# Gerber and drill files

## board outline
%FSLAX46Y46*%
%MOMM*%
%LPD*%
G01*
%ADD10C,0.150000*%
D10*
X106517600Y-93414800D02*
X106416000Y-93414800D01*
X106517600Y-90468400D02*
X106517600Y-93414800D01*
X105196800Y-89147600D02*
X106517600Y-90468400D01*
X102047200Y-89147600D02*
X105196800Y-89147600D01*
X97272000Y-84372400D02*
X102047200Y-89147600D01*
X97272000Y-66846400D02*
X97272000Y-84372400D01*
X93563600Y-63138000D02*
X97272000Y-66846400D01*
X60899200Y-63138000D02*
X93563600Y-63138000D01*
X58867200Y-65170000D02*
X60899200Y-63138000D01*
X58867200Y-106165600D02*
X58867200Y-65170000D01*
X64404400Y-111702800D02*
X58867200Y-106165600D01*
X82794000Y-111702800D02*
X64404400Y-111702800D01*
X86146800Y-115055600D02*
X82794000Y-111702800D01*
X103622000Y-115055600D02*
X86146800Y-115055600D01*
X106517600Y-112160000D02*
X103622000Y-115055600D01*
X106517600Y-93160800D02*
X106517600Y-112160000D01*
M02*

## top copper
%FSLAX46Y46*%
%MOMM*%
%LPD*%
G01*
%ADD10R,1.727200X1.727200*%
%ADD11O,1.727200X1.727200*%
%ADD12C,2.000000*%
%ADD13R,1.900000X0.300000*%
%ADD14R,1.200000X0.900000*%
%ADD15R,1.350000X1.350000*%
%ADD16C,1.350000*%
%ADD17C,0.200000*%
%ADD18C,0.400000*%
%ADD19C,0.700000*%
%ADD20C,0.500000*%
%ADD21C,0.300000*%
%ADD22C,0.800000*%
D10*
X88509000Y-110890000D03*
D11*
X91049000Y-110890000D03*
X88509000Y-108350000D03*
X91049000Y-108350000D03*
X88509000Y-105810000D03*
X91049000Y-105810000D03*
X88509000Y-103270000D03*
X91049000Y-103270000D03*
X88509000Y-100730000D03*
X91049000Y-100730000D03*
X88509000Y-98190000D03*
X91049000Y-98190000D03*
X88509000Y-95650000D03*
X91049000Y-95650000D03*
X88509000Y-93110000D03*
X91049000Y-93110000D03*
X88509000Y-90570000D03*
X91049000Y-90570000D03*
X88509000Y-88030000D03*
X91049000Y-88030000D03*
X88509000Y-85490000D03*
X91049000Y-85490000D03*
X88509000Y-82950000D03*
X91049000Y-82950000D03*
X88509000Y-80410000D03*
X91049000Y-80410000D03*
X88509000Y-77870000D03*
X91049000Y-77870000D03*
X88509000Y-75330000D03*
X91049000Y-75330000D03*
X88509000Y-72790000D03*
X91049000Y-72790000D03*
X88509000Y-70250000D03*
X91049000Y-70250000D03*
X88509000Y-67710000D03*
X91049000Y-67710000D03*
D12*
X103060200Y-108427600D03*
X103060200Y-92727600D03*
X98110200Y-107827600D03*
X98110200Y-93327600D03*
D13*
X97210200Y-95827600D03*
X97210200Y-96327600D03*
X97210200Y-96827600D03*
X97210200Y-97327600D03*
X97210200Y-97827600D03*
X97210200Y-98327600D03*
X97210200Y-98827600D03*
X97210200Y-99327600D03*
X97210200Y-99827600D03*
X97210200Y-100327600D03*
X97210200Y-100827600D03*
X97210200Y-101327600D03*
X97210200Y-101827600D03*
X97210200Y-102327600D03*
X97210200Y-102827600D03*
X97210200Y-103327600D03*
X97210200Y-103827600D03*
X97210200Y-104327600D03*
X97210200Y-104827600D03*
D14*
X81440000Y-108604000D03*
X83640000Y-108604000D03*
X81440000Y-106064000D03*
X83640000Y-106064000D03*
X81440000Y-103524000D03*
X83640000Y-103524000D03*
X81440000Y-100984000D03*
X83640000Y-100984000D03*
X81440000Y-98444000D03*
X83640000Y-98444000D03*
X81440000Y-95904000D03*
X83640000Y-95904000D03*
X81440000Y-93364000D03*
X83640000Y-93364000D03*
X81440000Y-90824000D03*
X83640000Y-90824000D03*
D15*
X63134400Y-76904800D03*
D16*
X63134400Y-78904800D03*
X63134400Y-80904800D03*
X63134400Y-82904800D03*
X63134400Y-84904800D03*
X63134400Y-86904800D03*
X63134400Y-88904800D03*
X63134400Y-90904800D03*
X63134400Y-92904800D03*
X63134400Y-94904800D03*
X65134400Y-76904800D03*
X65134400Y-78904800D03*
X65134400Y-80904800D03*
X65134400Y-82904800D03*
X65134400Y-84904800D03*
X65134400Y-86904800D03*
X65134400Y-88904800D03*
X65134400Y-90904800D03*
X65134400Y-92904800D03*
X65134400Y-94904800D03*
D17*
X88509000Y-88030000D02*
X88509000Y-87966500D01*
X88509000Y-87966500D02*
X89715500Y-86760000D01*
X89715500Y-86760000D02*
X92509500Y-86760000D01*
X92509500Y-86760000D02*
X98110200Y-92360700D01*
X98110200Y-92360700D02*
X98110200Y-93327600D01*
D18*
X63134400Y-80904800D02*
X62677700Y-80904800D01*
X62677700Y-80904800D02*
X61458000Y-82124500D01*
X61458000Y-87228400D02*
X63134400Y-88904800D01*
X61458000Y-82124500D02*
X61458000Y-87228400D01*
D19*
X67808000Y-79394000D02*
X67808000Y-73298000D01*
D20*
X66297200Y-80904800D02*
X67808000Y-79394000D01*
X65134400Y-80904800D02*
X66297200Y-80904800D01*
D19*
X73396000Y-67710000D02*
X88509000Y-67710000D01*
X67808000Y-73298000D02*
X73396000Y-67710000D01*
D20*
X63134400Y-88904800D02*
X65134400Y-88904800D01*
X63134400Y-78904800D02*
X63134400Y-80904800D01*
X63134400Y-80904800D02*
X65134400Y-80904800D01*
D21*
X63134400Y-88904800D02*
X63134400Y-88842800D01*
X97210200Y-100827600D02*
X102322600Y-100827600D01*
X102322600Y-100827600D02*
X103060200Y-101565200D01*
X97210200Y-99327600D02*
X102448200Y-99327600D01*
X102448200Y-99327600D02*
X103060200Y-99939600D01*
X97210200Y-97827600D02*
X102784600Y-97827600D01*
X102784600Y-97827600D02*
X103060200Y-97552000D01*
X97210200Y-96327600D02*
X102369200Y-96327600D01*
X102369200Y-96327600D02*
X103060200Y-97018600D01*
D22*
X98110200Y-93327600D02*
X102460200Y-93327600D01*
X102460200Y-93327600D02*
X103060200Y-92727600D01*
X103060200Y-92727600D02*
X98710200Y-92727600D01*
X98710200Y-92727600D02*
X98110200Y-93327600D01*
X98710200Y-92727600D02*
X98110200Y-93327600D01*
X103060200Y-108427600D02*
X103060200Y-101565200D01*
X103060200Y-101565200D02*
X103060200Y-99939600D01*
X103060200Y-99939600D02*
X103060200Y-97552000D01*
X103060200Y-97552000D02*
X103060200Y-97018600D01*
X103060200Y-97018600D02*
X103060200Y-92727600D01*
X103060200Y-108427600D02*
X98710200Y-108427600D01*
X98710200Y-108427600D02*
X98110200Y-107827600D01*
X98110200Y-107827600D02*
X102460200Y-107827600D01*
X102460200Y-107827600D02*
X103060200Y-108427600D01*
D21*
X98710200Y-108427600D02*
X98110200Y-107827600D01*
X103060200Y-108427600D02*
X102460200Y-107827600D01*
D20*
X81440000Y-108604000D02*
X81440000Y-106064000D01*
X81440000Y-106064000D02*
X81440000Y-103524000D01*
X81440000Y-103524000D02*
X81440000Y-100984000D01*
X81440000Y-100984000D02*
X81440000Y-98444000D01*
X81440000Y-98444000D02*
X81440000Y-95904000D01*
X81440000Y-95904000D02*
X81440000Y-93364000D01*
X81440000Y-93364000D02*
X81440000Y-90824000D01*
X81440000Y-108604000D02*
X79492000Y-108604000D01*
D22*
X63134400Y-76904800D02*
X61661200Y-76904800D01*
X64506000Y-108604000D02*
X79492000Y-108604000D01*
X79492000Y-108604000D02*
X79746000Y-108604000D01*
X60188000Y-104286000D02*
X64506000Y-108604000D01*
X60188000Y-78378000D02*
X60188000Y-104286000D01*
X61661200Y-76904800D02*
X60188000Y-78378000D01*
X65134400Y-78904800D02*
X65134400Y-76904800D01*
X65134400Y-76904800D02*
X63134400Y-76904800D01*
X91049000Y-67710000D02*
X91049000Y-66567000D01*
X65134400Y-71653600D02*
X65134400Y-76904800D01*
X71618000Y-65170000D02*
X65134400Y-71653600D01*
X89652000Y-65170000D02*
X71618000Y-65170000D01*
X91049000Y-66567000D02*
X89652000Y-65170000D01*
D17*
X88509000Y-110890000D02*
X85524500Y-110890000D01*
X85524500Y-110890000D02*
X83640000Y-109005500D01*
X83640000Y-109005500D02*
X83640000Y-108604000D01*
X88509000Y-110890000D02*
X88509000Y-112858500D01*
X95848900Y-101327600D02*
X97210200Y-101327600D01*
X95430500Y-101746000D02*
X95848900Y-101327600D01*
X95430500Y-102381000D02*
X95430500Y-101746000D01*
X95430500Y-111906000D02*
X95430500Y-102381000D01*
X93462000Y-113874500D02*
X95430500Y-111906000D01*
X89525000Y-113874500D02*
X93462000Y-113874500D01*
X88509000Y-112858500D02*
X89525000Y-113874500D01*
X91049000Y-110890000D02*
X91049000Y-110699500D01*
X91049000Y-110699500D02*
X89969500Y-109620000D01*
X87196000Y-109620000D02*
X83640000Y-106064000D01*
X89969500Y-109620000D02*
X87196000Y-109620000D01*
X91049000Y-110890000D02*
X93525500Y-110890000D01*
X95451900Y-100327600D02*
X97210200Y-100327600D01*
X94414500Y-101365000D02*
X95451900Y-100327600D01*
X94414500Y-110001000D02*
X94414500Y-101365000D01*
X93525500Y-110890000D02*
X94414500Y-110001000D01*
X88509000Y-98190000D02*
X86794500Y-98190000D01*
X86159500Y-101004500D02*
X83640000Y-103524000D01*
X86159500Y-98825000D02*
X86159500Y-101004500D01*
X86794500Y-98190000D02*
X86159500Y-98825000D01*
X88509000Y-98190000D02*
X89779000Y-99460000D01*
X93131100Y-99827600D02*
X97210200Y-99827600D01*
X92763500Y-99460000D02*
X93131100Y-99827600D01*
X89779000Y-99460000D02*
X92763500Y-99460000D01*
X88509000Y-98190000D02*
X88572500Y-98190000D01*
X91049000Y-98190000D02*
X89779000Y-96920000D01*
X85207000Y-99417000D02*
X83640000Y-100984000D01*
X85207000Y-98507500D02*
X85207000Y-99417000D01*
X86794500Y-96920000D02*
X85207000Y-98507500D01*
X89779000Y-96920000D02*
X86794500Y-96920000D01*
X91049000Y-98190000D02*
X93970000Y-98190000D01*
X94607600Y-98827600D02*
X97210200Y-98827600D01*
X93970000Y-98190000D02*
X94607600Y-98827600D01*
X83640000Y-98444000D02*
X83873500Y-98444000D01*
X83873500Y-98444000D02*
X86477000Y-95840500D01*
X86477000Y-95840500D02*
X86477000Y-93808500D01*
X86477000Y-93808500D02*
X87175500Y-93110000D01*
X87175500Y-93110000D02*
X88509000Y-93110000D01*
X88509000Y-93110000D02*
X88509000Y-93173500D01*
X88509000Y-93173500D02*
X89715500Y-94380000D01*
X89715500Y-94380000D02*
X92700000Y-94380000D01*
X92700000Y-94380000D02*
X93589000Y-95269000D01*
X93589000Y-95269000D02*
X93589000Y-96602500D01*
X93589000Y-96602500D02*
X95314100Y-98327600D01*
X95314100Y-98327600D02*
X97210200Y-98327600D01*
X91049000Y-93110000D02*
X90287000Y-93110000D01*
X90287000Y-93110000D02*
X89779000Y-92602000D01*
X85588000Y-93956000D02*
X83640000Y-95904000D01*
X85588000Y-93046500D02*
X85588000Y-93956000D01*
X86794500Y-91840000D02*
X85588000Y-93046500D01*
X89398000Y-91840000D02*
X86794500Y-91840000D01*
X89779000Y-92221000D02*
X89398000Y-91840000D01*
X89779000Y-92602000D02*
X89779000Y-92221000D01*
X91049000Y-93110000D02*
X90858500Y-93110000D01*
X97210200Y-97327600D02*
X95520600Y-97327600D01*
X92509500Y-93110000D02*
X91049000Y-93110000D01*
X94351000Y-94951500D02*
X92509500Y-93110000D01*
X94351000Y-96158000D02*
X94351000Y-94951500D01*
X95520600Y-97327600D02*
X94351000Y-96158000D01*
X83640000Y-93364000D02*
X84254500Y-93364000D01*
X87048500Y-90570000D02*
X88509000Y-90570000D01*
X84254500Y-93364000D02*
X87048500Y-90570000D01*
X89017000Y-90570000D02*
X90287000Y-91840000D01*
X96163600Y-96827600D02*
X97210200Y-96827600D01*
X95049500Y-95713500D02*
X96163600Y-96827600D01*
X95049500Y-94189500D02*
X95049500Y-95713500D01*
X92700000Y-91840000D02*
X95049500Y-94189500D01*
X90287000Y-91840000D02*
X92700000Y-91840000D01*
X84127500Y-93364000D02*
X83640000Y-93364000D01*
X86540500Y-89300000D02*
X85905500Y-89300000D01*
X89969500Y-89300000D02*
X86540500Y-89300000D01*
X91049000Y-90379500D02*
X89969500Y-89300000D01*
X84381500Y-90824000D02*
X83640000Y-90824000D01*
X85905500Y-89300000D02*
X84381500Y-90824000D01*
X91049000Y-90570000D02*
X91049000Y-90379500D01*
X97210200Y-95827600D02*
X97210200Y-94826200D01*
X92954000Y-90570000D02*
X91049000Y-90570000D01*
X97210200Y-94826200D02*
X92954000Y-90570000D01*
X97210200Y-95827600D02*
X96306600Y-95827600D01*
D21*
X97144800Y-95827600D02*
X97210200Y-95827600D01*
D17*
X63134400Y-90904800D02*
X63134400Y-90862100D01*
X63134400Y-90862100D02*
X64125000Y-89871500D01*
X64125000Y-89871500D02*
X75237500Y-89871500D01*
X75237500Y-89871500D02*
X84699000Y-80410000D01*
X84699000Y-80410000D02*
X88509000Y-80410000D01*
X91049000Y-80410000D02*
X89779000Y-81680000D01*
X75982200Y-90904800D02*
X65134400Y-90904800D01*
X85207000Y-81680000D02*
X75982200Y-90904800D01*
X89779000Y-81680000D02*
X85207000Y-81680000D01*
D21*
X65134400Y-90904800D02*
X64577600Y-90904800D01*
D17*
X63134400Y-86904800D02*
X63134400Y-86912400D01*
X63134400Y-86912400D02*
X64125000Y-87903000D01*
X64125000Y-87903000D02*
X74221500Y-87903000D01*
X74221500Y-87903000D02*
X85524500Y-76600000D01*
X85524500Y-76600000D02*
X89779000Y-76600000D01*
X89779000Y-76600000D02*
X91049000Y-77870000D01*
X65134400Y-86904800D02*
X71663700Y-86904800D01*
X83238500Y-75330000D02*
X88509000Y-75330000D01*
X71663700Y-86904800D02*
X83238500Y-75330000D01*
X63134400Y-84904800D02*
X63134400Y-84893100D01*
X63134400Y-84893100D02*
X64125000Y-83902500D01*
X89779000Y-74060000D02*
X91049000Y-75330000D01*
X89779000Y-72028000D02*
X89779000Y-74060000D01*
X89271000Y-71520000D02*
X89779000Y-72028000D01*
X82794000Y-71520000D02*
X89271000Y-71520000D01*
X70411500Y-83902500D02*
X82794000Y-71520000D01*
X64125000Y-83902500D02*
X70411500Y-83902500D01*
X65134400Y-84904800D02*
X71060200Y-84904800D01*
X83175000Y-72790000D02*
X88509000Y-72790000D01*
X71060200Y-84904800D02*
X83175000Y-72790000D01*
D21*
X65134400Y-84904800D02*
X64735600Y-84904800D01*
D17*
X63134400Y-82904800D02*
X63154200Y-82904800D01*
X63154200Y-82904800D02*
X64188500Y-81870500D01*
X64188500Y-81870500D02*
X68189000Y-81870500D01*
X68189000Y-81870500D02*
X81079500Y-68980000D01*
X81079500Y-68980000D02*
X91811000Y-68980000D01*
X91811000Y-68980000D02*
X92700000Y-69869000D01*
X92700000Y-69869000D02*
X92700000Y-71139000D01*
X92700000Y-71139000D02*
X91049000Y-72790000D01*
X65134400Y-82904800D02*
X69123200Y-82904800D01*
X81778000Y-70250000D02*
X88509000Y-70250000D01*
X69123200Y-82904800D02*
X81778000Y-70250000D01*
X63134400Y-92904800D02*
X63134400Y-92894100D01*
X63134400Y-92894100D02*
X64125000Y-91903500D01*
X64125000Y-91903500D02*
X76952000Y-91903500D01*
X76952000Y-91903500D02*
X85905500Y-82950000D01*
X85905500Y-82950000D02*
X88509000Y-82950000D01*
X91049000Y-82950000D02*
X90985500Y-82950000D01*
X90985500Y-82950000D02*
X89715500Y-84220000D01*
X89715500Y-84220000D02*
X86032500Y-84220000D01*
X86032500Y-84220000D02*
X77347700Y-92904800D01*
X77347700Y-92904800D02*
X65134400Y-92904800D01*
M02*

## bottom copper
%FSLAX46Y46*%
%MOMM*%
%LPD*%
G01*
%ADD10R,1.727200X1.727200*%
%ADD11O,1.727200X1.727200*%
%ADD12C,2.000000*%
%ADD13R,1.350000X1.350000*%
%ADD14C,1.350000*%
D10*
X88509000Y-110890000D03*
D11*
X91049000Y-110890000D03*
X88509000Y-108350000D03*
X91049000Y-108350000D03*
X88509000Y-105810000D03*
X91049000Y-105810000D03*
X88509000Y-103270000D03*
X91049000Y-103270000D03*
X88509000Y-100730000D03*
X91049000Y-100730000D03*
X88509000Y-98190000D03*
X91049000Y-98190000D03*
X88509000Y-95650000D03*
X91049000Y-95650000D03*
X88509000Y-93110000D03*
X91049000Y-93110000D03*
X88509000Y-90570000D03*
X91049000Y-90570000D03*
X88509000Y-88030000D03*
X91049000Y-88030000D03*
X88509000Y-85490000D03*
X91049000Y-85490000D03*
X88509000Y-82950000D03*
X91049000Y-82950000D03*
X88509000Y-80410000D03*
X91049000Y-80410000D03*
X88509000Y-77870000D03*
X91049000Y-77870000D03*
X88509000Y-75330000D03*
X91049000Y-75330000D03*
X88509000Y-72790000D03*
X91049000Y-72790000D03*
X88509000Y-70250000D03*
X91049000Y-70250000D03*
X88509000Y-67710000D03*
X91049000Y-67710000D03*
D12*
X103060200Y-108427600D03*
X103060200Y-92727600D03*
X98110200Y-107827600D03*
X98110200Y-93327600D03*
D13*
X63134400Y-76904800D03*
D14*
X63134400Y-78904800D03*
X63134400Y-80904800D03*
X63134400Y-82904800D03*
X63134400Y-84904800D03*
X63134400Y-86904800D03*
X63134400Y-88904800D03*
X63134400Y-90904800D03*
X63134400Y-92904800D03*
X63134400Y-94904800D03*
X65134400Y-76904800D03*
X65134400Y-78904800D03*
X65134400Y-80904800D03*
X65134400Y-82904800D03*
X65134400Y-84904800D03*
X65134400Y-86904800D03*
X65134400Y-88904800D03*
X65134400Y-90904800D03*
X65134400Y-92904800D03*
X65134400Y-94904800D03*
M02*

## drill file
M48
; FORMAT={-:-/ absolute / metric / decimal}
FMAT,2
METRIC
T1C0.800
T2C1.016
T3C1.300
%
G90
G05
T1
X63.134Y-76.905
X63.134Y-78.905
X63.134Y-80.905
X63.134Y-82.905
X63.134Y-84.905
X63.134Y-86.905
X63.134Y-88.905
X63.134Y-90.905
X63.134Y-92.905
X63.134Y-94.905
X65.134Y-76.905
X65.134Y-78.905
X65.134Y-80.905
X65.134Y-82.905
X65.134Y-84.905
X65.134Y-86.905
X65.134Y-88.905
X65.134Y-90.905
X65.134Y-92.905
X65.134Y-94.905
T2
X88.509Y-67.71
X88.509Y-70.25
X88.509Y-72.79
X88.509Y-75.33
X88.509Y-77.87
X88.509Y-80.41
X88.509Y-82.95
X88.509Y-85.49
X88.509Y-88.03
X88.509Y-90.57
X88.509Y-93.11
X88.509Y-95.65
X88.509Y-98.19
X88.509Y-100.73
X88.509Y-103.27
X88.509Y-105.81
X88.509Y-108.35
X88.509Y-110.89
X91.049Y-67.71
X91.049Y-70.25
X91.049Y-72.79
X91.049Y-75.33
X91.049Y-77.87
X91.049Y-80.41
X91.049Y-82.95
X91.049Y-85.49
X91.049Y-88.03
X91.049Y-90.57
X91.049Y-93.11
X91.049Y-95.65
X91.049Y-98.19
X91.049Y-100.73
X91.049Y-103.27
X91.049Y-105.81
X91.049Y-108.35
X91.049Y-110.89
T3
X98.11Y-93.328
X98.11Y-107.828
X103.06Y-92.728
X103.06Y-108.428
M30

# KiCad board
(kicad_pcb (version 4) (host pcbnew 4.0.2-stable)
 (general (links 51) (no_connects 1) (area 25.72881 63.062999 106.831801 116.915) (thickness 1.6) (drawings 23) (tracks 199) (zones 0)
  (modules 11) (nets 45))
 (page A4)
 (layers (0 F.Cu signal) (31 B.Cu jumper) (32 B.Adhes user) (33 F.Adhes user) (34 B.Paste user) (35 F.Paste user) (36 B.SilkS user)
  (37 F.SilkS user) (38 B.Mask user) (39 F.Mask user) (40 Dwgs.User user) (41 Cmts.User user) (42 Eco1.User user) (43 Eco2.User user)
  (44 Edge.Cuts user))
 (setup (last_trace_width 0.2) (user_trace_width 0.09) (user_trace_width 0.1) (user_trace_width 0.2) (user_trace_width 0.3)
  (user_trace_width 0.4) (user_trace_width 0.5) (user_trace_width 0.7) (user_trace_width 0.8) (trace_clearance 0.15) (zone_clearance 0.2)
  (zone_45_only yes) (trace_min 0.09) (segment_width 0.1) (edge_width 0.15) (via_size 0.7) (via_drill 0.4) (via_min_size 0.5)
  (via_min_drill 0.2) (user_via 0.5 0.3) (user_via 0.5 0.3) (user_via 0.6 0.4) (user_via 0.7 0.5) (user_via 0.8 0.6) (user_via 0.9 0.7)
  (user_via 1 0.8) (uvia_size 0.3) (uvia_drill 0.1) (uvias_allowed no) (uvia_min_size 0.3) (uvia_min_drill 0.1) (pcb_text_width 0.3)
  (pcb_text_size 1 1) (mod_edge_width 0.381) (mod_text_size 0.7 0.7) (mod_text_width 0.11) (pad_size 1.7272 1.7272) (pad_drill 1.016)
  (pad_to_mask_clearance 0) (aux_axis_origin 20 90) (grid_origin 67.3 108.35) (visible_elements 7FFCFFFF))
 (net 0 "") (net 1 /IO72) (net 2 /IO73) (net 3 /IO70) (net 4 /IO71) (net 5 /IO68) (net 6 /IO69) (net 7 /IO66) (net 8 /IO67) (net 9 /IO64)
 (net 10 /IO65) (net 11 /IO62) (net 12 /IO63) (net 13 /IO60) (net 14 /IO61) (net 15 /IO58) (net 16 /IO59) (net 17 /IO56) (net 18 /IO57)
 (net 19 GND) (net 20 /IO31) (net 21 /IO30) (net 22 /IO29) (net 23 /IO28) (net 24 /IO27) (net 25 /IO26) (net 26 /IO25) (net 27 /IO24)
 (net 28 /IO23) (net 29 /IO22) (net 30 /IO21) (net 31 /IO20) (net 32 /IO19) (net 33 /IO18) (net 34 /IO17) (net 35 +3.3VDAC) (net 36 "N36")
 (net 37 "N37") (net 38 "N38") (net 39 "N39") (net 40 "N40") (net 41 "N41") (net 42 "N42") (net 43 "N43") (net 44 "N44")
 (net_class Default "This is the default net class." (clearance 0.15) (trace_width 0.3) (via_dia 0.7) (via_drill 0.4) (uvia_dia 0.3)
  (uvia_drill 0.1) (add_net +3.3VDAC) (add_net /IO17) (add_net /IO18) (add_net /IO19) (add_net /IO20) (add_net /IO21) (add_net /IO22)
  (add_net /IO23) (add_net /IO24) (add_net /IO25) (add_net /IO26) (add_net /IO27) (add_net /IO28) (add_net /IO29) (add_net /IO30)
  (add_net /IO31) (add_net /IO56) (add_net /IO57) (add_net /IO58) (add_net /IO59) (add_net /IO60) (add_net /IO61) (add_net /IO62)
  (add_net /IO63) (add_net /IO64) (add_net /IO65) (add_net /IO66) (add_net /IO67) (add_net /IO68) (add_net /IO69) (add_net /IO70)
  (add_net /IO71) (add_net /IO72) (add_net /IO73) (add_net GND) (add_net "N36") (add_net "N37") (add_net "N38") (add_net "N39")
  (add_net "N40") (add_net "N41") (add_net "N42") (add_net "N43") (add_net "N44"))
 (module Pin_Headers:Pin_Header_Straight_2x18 (layer B.Cu) (at 88.509 110.89)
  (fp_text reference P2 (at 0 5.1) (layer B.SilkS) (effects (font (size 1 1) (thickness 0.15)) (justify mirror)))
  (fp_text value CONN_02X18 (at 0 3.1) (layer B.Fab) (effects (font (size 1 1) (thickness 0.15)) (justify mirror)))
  (pad 1 thru_hole rect (at 0 0) (size 1.7272 1.7272) (drill 1.016) (layers *.Cu *.Mask) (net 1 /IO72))
  (pad 2 thru_hole oval (at 2.54 0) (size 1.7272 1.7272) (drill 1.016) (layers *.Cu *.Mask) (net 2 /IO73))
  (pad 3 thru_hole oval (at 0 -2.54) (size 1.7272 1.7272) (drill 1.016) (layers *.Cu *.Mask) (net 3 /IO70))
  (pad 4 thru_hole oval (at 2.54 -2.54) (size 1.7272 1.7272) (drill 1.016) (layers *.Cu *.Mask) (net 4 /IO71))
  (pad 5 thru_hole oval (at 0 -5.08) (size 1.7272 1.7272) (drill 1.016) (layers *.Cu *.Mask) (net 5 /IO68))
  (pad 6 thru_hole oval (at 2.54 -5.08) (size 1.7272 1.7272) (drill 1.016) (layers *.Cu *.Mask) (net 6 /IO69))
  (pad 7 thru_hole oval (at 0 -7.62) (size 1.7272 1.7272) (drill 1.016) (layers *.Cu *.Mask) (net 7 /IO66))
  (pad 8 thru_hole oval (at 2.54 -7.62) (size 1.7272 1.7272) (drill 1.016) (layers *.Cu *.Mask) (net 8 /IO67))
  (pad 9 thru_hole oval (at 0 -10.16) (size 1.7272 1.7272) (drill 1.016) (layers *.Cu *.Mask) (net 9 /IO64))
  (pad 10 thru_hole oval (at 2.54 -10.16) (size 1.7272 1.7272) (drill 1.016) (layers *.Cu *.Mask) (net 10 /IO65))
  (pad 11 thru_hole oval (at 0 -12.7) (size 1.7272 1.7272) (drill 1.016) (layers *.Cu *.Mask) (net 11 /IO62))
  (pad 12 thru_hole oval (at 2.54 -12.7) (size 1.7272 1.7272) (drill 1.016) (layers *.Cu *.Mask) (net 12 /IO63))
  (pad 13 thru_hole oval (at 0 -15.24) (size 1.7272 1.7272) (drill 1.016) (layers *.Cu *.Mask) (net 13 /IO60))
  (pad 14 thru_hole oval (at 2.54 -15.24) (size 1.7272 1.7272) (drill 1.016) (layers *.Cu *.Mask) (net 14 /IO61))
  (pad 15 thru_hole oval (at 0 -17.78) (size 1.7272 1.7272) (drill 1.016) (layers *.Cu *.Mask) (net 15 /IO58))
  (pad 16 thru_hole oval (at 2.54 -17.78) (size 1.7272 1.7272) (drill 1.016) (layers *.Cu *.Mask) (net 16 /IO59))
  (pad 17 thru_hole oval (at 0 -20.32) (size 1.7272 1.7272) (drill 1.016) (layers *.Cu *.Mask) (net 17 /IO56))
  (pad 18 thru_hole oval (at 2.54 -20.32) (size 1.7272 1.7272) (drill 1.016) (layers *.Cu *.Mask) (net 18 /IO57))
  (pad 19 thru_hole oval (at 0 -22.86) (size 1.7272 1.7272) (drill 1.016) (layers *.Cu *.Mask) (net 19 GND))
  (pad 20 thru_hole oval (at 2.54 -22.86) (size 1.7272 1.7272) (drill 1.016) (layers *.Cu *.Mask) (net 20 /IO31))
  (pad 21 thru_hole oval (at 0 -25.4) (size 1.7272 1.7272) (drill 1.016) (layers *.Cu *.Mask) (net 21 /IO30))
  (pad 22 thru_hole oval (at 2.54 -25.4) (size 1.7272 1.7272) (drill 1.016) (layers *.Cu *.Mask) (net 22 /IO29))
  (pad 23 thru_hole oval (at 0 -27.94) (size 1.7272 1.7272) (drill 1.016) (layers *.Cu *.Mask) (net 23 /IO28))
  (pad 24 thru_hole oval (at 2.54 -27.94) (size 1.7272 1.7272) (drill 1.016) (layers *.Cu *.Mask) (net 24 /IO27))
  (pad 25 thru_hole oval (at 0 -30.48) (size 1.7272 1.7272) (drill 1.016) (layers *.Cu *.Mask) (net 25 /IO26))
  (pad 26 thru_hole oval (at 2.54 -30.48) (size 1.7272 1.7272) (drill 1.016) (layers *.Cu *.Mask) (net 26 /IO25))
  (pad 27 thru_hole oval (at 0 -33.02) (size 1.7272 1.7272) (drill 1.016) (layers *.Cu *.Mask) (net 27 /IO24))
  (pad 28 thru_hole oval (at 2.54 -33.02) (size 1.7272 1.7272) (drill 1.016) (layers *.Cu *.Mask) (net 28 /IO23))
  (pad 29 thru_hole oval (at 0 -35.56) (size 1.7272 1.7272) (drill 1.016) (layers *.Cu *.Mask) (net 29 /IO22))
  (pad 30 thru_hole oval (at 2.54 -35.56) (size 1.7272 1.7272) (drill 1.016) (layers *.Cu *.Mask) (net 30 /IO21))
  (pad 31 thru_hole oval (at 0 -38.1) (size 1.7272 1.7272) (drill 1.016) (layers *.Cu *.Mask) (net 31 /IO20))
  (pad 32 thru_hole oval (at 2.54 -38.1) (size 1.7272 1.7272) (drill 1.016) (layers *.Cu *.Mask) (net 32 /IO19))
  (pad 33 thru_hole oval (at 0 -40.64) (size 1.7272 1.7272) (drill 1.016) (layers *.Cu *.Mask) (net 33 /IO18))
  (pad 34 thru_hole oval (at 2.54 -40.64) (size 1.7272 1.7272) (drill 1.016) (layers *.Cu *.Mask) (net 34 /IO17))
  (pad 35 thru_hole oval (at 0 -43.18) (size 1.7272 1.7272) (drill 1.016) (layers *.Cu *.Mask) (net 19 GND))
  (pad 36 thru_hole oval (at 2.54 -43.18) (size 1.7272 1.7272) (drill 1.016) (layers *.Cu *.Mask) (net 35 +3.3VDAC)))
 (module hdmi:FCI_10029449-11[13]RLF (layer F.Cu) (at 98.1102 100.5776 90)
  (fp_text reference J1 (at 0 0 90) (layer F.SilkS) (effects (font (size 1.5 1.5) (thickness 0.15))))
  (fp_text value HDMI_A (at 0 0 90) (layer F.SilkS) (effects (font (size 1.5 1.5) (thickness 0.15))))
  (pad SHLD thru_hole circle (at -7.85 4.95 90) (size 2 2) (drill 1.3) (layers *.Cu *.SilkS *.Mask) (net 19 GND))
  (pad SHLD thru_hole circle (at 7.85 4.95 90) (size 2 2) (drill 1.3) (layers *.Cu *.SilkS *.Mask) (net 19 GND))
  (pad SHLD thru_hole circle (at -7.25 0 90) (size 2 2) (drill 1.3) (layers *.Cu *.SilkS *.Mask) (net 19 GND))
  (pad SHLD thru_hole circle (at 7.25 0 90) (size 2 2) (drill 1.3) (layers *.Cu *.SilkS *.Mask) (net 19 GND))
  (pad 1 smd rect (at 4.75 -0.9 90) (size 0.3 1.9) (layers F.Cu F.Paste F.Mask) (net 18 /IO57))
  (pad 2 smd rect (at 4.25 -0.9 90) (size 0.3 1.9) (layers F.Cu F.Paste F.Mask) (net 19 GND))
  (pad 3 smd rect (at 3.75 -0.9 90) (size 0.3 1.9) (layers F.Cu F.Paste F.Mask) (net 17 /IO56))
  (pad 4 smd rect (at 3.25 -0.9 90) (size 0.3 1.9) (layers F.Cu F.Paste F.Mask) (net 16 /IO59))
  (pad 5 smd rect (at 2.75 -0.9 90) (size 0.3 1.9) (layers F.Cu F.Paste F.Mask) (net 19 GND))
  (pad 6 smd rect (at 2.25 -0.9 90) (size 0.3 1.9) (layers F.Cu F.Paste F.Mask) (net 15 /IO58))
  (pad 7 smd rect (at 1.75 -0.9 90) (size 0.3 1.9) (layers F.Cu F.Paste F.Mask) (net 12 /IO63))
  (pad 8 smd rect (at 1.25 -0.9 90) (size 0.3 1.9) (layers F.Cu F.Paste F.Mask) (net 19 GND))
  (pad 9 smd rect (at 0.75 -0.9 90) (size 0.3 1.9) (layers F.Cu F.Paste F.Mask) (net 11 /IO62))
  (pad 10 smd rect (at 0.25 -0.9 90) (size 0.3 1.9) (layers F.Cu F.Paste F.Mask) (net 2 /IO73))
  (pad 11 smd rect (at -0.25 -0.9 90) (size 0.3 1.9) (layers F.Cu F.Paste F.Mask) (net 19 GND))
  (pad 12 smd rect (at -0.75 -0.9 90) (size 0.3 1.9) (layers F.Cu F.Paste F.Mask) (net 1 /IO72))
  (pad 13 smd rect (at -1.25 -0.9 90) (size 0.3 1.9) (layers F.Cu F.Paste F.Mask) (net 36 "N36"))
  (pad 14 smd rect (at -1.75 -0.9 90) (size 0.3 1.9) (layers F.Cu F.Paste F.Mask) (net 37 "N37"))
  (pad 15 smd rect (at -2.25 -0.9 90) (size 0.3 1.9) (layers F.Cu F.Paste F.Mask) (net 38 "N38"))
  (pad 16 smd rect (at -2.75 -0.9 90) (size 0.3 1.9) (layers F.Cu F.Paste F.Mask) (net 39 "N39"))
  (pad 17 smd rect (at -3.25 -0.9 90) (size 0.3 1.9) (layers F.Cu F.Paste F.Mask) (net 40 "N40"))
  (pad 18 smd rect (at -3.75 -0.9 90) (size 0.3 1.9) (layers F.Cu F.Paste F.Mask) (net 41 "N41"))
  (pad 19 smd rect (at -4.25 -0.9 90) (size 0.3 1.9) (layers F.Cu F.Paste F.Mask) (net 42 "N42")))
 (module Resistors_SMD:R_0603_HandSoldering (layer F.Cu) (at 82.54 108.604)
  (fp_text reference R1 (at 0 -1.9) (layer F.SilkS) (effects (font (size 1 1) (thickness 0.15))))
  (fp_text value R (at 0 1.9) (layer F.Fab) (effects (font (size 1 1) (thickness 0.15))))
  (pad 1 smd rect (at -1.1 0) (size 1.2 0.9) (layers F.Cu F.Paste F.Mask) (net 35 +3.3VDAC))
  (pad 2 smd rect (at 1.1 0) (size 1.2 0.9) (layers F.Cu F.Paste F.Mask) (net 1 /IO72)))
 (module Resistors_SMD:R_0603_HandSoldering (layer F.Cu) (at 82.54 106.064)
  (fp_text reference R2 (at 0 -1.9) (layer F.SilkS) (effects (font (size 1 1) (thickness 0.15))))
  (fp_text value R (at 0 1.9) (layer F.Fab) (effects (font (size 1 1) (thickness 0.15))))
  (pad 1 smd rect (at -1.1 0) (size 1.2 0.9) (layers F.Cu F.Paste F.Mask) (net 35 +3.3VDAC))
  (pad 2 smd rect (at 1.1 0) (size 1.2 0.9) (layers F.Cu F.Paste F.Mask) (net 2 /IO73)))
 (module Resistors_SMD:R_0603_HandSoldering (layer F.Cu) (at 82.54 103.524)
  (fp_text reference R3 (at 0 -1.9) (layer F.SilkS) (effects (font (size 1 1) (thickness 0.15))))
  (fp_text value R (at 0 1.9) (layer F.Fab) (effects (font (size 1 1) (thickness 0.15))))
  (pad 1 smd rect (at -1.1 0) (size 1.2 0.9) (layers F.Cu F.Paste F.Mask) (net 35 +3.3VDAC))
  (pad 2 smd rect (at 1.1 0) (size 1.2 0.9) (layers F.Cu F.Paste F.Mask) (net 11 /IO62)))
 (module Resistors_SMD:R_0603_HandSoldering (layer F.Cu) (at 82.54 100.984)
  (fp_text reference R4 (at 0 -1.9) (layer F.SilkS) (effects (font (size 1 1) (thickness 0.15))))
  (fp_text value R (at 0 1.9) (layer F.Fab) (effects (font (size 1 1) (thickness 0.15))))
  (pad 1 smd rect (at -1.1 0) (size 1.2 0.9) (layers F.Cu F.Paste F.Mask) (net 35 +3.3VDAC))
  (pad 2 smd rect (at 1.1 0) (size 1.2 0.9) (layers F.Cu F.Paste F.Mask) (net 12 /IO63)))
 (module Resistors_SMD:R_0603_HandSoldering (layer F.Cu) (at 82.54 98.444)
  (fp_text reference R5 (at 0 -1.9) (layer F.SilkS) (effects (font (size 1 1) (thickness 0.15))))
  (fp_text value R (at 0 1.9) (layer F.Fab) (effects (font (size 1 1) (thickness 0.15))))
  (pad 1 smd rect (at -1.1 0) (size 1.2 0.9) (layers F.Cu F.Paste F.Mask) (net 35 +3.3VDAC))
  (pad 2 smd rect (at 1.1 0) (size 1.2 0.9) (layers F.Cu F.Paste F.Mask) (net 15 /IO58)))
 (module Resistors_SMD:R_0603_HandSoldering (layer F.Cu) (at 82.54 95.904)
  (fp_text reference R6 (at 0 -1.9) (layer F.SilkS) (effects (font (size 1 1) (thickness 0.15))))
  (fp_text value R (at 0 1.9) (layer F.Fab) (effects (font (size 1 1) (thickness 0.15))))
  (pad 1 smd rect (at -1.1 0) (size 1.2 0.9) (layers F.Cu F.Paste F.Mask) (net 35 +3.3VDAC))
  (pad 2 smd rect (at 1.1 0) (size 1.2 0.9) (layers F.Cu F.Paste F.Mask) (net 16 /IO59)))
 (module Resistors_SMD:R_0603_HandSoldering (layer F.Cu) (at 82.54 93.364)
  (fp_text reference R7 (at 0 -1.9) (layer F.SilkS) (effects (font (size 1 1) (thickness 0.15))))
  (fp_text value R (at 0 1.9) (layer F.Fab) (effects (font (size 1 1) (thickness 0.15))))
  (pad 1 smd rect (at -1.1 0) (size 1.2 0.9) (layers F.Cu F.Paste F.Mask) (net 35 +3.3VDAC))
  (pad 2 smd rect (at 1.1 0) (size 1.2 0.9) (layers F.Cu F.Paste F.Mask) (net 17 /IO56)))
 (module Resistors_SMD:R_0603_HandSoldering (layer F.Cu) (at 82.54 90.824)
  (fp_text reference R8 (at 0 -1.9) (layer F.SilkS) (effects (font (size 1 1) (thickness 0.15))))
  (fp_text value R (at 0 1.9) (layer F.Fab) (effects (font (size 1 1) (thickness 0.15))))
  (pad 1 smd rect (at -1.1 0) (size 1.2 0.9) (layers F.Cu F.Paste F.Mask) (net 35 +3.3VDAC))
  (pad 2 smd rect (at 1.1 0) (size 1.2 0.9) (layers F.Cu F.Paste F.Mask) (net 18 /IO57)))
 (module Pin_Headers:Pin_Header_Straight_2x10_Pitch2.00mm (layer F.Cu) (at 63.1344 76.9048)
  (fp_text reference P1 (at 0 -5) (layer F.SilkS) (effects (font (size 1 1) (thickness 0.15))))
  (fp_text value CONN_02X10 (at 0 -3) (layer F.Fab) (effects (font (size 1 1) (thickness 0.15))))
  (pad 1 thru_hole rect (at 0 0) (size 1.35 1.35) (drill 0.8) (layers *.Cu *.Mask) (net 35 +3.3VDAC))
  (pad 3 thru_hole circle (at 0 2) (size 1.35 1.35) (drill 0.8) (layers *.Cu *.Mask) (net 19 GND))
  (pad 5 thru_hole circle (at 0 4) (size 1.35 1.35) (drill 0.8) (layers *.Cu *.Mask) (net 19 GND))
  (pad 7 thru_hole circle (at 0 6) (size 1.35 1.35) (drill 0.8) (layers *.Cu *.Mask) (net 32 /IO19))
  (pad 9 thru_hole circle (at 0 8) (size 1.35 1.35) (drill 0.8) (layers *.Cu *.Mask) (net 30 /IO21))
  (pad 11 thru_hole circle (at 0 10) (size 1.35 1.35) (drill 0.8) (layers *.Cu *.Mask) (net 28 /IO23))
  (pad 13 thru_hole circle (at 0 12) (size 1.35 1.35) (drill 0.8) (layers *.Cu *.Mask) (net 19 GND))
  (pad 15 thru_hole circle (at 0 14) (size 1.35 1.35) (drill 0.8) (layers *.Cu *.Mask) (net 25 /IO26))
  (pad 17 thru_hole circle (at 0 16) (size 1.35 1.35) (drill 0.8) (layers *.Cu *.Mask) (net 23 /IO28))
  (pad 19 thru_hole circle (at 0 18) (size 1.35 1.35) (drill 0.8) (layers *.Cu *.Mask) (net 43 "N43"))
  (pad 2 thru_hole circle (at 2 0) (size 1.35 1.35) (drill 0.8) (layers *.Cu *.Mask) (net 35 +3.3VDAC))
  (pad 4 thru_hole circle (at 2 2) (size 1.35 1.35) (drill 0.8) (layers *.Cu *.Mask) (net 35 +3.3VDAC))
  (pad 6 thru_hole circle (at 2 4) (size 1.35 1.35) (drill 0.8) (layers *.Cu *.Mask) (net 19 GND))
  (pad 8 thru_hole circle (at 2 6) (size 1.35 1.35) (drill 0.8) (layers *.Cu *.Mask) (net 33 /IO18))
  (pad 10 thru_hole circle (at 2 8) (size 1.35 1.35) (drill 0.8) (layers *.Cu *.Mask) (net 31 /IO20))
  (pad 12 thru_hole circle (at 2 10) (size 1.35 1.35) (drill 0.8) (layers *.Cu *.Mask) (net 29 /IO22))
  (pad 14 thru_hole circle (at 2 12) (size 1.35 1.35) (drill 0.8) (layers *.Cu *.Mask) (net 19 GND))
  (pad 16 thru_hole circle (at 2 14) (size 1.35 1.35) (drill 0.8) (layers *.Cu *.Mask) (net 26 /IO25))
  (pad 18 thru_hole circle (at 2 16) (size 1.35 1.35) (drill 0.8) (layers *.Cu *.Mask) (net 24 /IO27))
  (pad 20 thru_hole circle (at 2 18) (size 1.35 1.35) (drill 0.8) (layers *.Cu *.Mask) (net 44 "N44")))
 (gr_line (start 106.5176 93.4148) (end 106.416 93.4148) (angle 90) (layer Edge.Cuts) (width 0.15))
 (gr_line (start 106.5176 90.4684) (end 106.5176 93.4148) (angle 90) (layer Edge.Cuts) (width 0.15))
 (gr_line (start 105.1968 89.1476) (end 106.5176 90.4684) (angle 90) (layer Edge.Cuts) (width 0.15))
 (gr_line (start 102.0472 89.1476) (end 105.1968 89.1476) (angle 90) (layer Edge.Cuts) (width 0.15))
 (gr_line (start 97.272 84.3724) (end 102.0472 89.1476) (angle 90) (layer Edge.Cuts) (width 0.15))
 (gr_line (start 97.272 66.8464) (end 97.272 84.3724) (angle 90) (layer Edge.Cuts) (width 0.15))
 (gr_line (start 93.5636 63.138) (end 97.272 66.8464) (angle 90) (layer Edge.Cuts) (width 0.15))
 (gr_line (start 60.8992 63.138) (end 93.5636 63.138) (angle 90) (layer Edge.Cuts) (width 0.15))
 (gr_line (start 58.8672 65.17) (end 60.8992 63.138) (angle 90) (layer Edge.Cuts) (width 0.15))
 (gr_line (start 58.8672 106.1656) (end 58.8672 65.17) (angle 90) (layer Edge.Cuts) (width 0.15))
 (gr_line (start 64.4044 111.7028) (end 58.8672 106.1656) (angle 90) (layer Edge.Cuts) (width 0.15))
 (gr_line (start 82.794 111.7028) (end 64.4044 111.7028) (angle 90) (layer Edge.Cuts) (width 0.15))
 (gr_line (start 86.1468 115.0556) (end 82.794 111.7028) (angle 90) (layer Edge.Cuts) (width 0.15))
 (gr_line (start 103.622 115.0556) (end 86.1468 115.0556) (angle 90) (layer Edge.Cuts) (width 0.15))
 (gr_line (start 106.5176 112.16) (end 103.622 115.0556) (angle 90) (layer Edge.Cuts) (width 0.15))
 (gr_line (start 106.5176 93.1608) (end 106.5176 112.16) (angle 90) (layer Edge.Cuts) (width 0.15))
 (segment (start 88.509 88.03) (end 88.509 87.9665) (width 0.2) (layer F.Cu) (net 19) (status C00000))
 (segment (start 88.509 87.9665) (end 89.7155 86.76) (width 0.2) (layer F.Cu) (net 19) (status 400000))
 (segment (start 89.7155 86.76) (end 92.5095 86.76) (width 0.2) (layer F.Cu) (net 19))
 (segment (start 92.5095 86.76) (end 98.1102 92.3607) (width 0.2) (layer F.Cu) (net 19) (status 800000))
 (segment (start 98.1102 92.3607) (end 98.1102 93.3276) (width 0.2) (layer F.Cu) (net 19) (status C00000))
 (segment (start 63.1344 80.9048) (end 62.6777 80.9048) (width 0.4) (layer F.Cu) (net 19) (status C00000))
 (segment (start 62.6777 80.9048) (end 61.458 82.1245) (width 0.4) (layer F.Cu) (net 19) (status 400000))
 (segment (start 61.458 87.2284) (end 63.1344 88.9048) (width 0.4) (layer F.Cu) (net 19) (status 800000))
 (segment (start 61.458 82.1245) (end 61.458 87.2284) (width 0.4) (layer F.Cu) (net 19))
 (segment (start 67.808 79.394) (end 67.808 73.298) (width 0.7) (layer F.Cu) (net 19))
 (segment (start 66.2972 80.9048) (end 67.808 79.394) (width 0.5) (layer F.Cu) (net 19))
 (segment (start 65.1344 80.9048) (end 66.2972 80.9048) (width 0.5) (layer F.Cu) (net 19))
 (segment (start 73.396 67.71) (end 88.509 67.71) (width 0.7) (layer F.Cu) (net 19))
 (segment (start 67.808 73.298) (end 73.396 67.71) (width 0.7) (layer F.Cu) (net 19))
 (segment (start 63.1344 88.9048) (end 65.1344 88.9048) (width 0.5) (layer F.Cu) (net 19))
 (segment (start 63.1344 78.9048) (end 63.1344 80.9048) (width 0.5) (layer F.Cu) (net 19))
 (segment (start 63.1344 80.9048) (end 65.1344 80.9048) (width 0.5) (layer F.Cu) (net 19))
 (segment (start 63.1344 88.9048) (end 63.1344 88.8428) (width 0.3) (layer F.Cu) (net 19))
 (segment (start 97.2102 100.8276) (end 102.3226 100.8276) (width 0.3) (layer F.Cu) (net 19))
 (segment (start 102.3226 100.8276) (end 103.0602 101.5652) (width 0.3) (layer F.Cu) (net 19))
 (segment (start 97.2102 99.3276) (end 102.4482 99.3276) (width 0.3) (layer F.Cu) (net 19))
 (segment (start 102.4482 99.3276) (end 103.0602 99.9396) (width 0.3) (layer F.Cu) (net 19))
 (segment (start 97.2102 97.8276) (end 102.7846 97.8276) (width 0.3) (layer F.Cu) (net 19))
 (segment (start 102.7846 97.8276) (end 103.0602 97.552) (width 0.3) (layer F.Cu) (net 19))
 (segment (start 97.2102 96.3276) (end 102.3692 96.3276) (width 0.3) (layer F.Cu) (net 19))
 (segment (start 102.3692 96.3276) (end 103.0602 97.0186) (width 0.3) (layer F.Cu) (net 19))
 (segment (start 98.1102 93.3276) (end 102.4602 93.3276) (width 0.8) (layer F.Cu) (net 19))
 (segment (start 102.4602 93.3276) (end 103.0602 92.7276) (width 0.8) (layer F.Cu) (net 19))
 (segment (start 103.0602 92.7276) (end 98.7102 92.7276) (width 0.8) (layer F.Cu) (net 19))
 (segment (start 98.7102 92.7276) (end 98.1102 93.3276) (width 0.8) (layer F.Cu) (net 19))
 (segment (start 98.7102 92.7276) (end 98.1102 93.3276) (width 0.8) (layer F.Cu) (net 19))
 (segment (start 103.0602 108.4276) (end 103.0602 101.5652) (width 0.8) (layer F.Cu) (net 19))
 (segment (start 103.0602 101.5652) (end 103.0602 99.9396) (width 0.8) (layer F.Cu) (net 19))
 (segment (start 103.0602 99.9396) (end 103.0602 97.552) (width 0.8) (layer F.Cu) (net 19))
 (segment (start 103.0602 97.552) (end 103.0602 97.0186) (width 0.8) (layer F.Cu) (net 19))
 (segment (start 103.0602 97.0186) (end 103.0602 92.7276) (width 0.8) (layer F.Cu) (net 19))
 (segment (start 103.0602 108.4276) (end 98.7102 108.4276) (width 0.8) (layer F.Cu) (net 19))
 (segment (start 98.7102 108.4276) (end 98.1102 107.8276) (width 0.8) (layer F.Cu) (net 19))
 (segment (start 98.1102 107.8276) (end 102.4602 107.8276) (width 0.8) (layer F.Cu) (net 19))
 (segment (start 102.4602 107.8276) (end 103.0602 108.4276) (width 0.8) (layer F.Cu) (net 19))
 (segment (start 98.7102 108.4276) (end 98.1102 107.8276) (width 0.3) (layer F.Cu) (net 19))
 (segment (start 103.0602 108.4276) (end 102.4602 107.8276) (width 0.3) (layer F.Cu) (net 19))
 (segment (start 81.44 108.604) (end 81.44 106.064) (width 0.5) (layer F.Cu) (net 35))
 (segment (start 81.44 106.064) (end 81.44 103.524) (width 0.5) (layer F.Cu) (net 35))
 (segment (start 81.44 103.524) (end 81.44 100.984) (width 0.5) (layer F.Cu) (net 35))
 (segment (start 81.44 100.984) (end 81.44 98.444) (width 0.5) (layer F.Cu) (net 35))
 (segment (start 81.44 98.444) (end 81.44 95.904) (width 0.5) (layer F.Cu) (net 35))
 (segment (start 81.44 95.904) (end 81.44 93.364) (width 0.5) (layer F.Cu) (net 35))
 (segment (start 81.44 93.364) (end 81.44 90.824) (width 0.5) (layer F.Cu) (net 35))
 (segment (start 81.44 108.604) (end 79.492 108.604) (width 0.5) (layer F.Cu) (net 35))
 (segment (start 63.1344 76.9048) (end 61.6612 76.9048) (width 0.8) (layer F.Cu) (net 35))
 (segment (start 64.506 108.604) (end 79.492 108.604) (width 0.8) (layer F.Cu) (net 35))
 (segment (start 79.492 108.604) (end 79.746 108.604) (width 0.8) (layer F.Cu) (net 35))
 (segment (start 60.188 104.286) (end 64.506 108.604) (width 0.8) (layer F.Cu) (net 35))
 (segment (start 60.188 78.378) (end 60.188 104.286) (width 0.8) (layer F.Cu) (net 35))
 (segment (start 61.6612 76.9048) (end 60.188 78.378) (width 0.8) (layer F.Cu) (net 35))
 (segment (start 65.1344 78.9048) (end 65.1344 76.9048) (width 0.8) (layer F.Cu) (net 35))
 (segment (start 65.1344 76.9048) (end 63.1344 76.9048) (width 0.8) (layer F.Cu) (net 35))
 (segment (start 91.049 67.71) (end 91.049 66.567) (width 0.8) (layer F.Cu) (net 35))
 (segment (start 65.1344 71.6536) (end 65.1344 76.9048) (width 0.8) (layer F.Cu) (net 35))
 (segment (start 71.618 65.17) (end 65.1344 71.6536) (width 0.8) (layer F.Cu) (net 35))
 (segment (start 89.652 65.17) (end 71.618 65.17) (width 0.8) (layer F.Cu) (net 35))
 (segment (start 91.049 66.567) (end 89.652 65.17) (width 0.8) (layer F.Cu) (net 35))
 (segment (start 88.509 110.89) (end 85.5245 110.89) (width 0.2) (layer F.Cu) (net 1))
 (segment (start 85.5245 110.89) (end 83.64 109.0055) (width 0.2) (layer F.Cu) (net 1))
 (segment (start 83.64 109.0055) (end 83.64 108.604) (width 0.2) (layer F.Cu) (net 1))
 (segment (start 88.509 110.89) (end 88.509 112.8585) (width 0.2) (layer F.Cu) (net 1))
 (segment (start 95.8489 101.3276) (end 97.2102 101.3276) (width 0.2) (layer F.Cu) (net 1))
 (segment (start 95.4305 101.746) (end 95.8489 101.3276) (width 0.2) (layer F.Cu) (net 1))
 (segment (start 95.4305 102.381) (end 95.4305 101.746) (width 0.2) (layer F.Cu) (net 1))
 (segment (start 95.4305 111.906) (end 95.4305 102.381) (width 0.2) (layer F.Cu) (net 1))
 (segment (start 93.462 113.8745) (end 95.4305 111.906) (width 0.2) (layer F.Cu) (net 1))
 (segment (start 89.525 113.8745) (end 93.462 113.8745) (width 0.2) (layer F.Cu) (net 1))
 (segment (start 88.509 112.8585) (end 89.525 113.8745) (width 0.2) (layer F.Cu) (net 1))
 (segment (start 91.049 110.89) (end 91.049 110.6995) (width 0.2) (layer F.Cu) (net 2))
 (segment (start 91.049 110.6995) (end 89.9695 109.62) (width 0.2) (layer F.Cu) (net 2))
 (segment (start 87.196 109.62) (end 83.64 106.064) (width 0.2) (layer F.Cu) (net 2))
 (segment (start 89.9695 109.62) (end 87.196 109.62) (width 0.2) (layer F.Cu) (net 2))
 (segment (start 91.049 110.89) (end 93.5255 110.89) (width 0.2) (layer F.Cu) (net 2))
 (segment (start 95.4519 100.3276) (end 97.2102 100.3276) (width 0.2) (layer F.Cu) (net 2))
 (segment (start 94.4145 101.365) (end 95.4519 100.3276) (width 0.2) (layer F.Cu) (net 2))
 (segment (start 94.4145 110.001) (end 94.4145 101.365) (width 0.2) (layer F.Cu) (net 2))
 (segment (start 93.5255 110.89) (end 94.4145 110.001) (width 0.2) (layer F.Cu) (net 2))
 (segment (start 88.509 98.19) (end 86.7945 98.19) (width 0.2) (layer F.Cu) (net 11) (status 400000))
 (segment (start 86.1595 101.0045) (end 83.64 103.524) (width 0.2) (layer F.Cu) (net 11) (status 800000))
 (segment (start 86.1595 98.825) (end 86.1595 101.0045) (width 0.2) (layer F.Cu) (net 11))
 (segment (start 86.7945 98.19) (end 86.1595 98.825) (width 0.2) (layer F.Cu) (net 11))
 (segment (start 88.509 98.19) (end 89.779 99.46) (width 0.2) (layer F.Cu) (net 11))
 (segment (start 93.1311 99.8276) (end 97.2102 99.8276) (width 0.2) (layer F.Cu) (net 11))
 (segment (start 92.7635 99.46) (end 93.1311 99.8276) (width 0.2) (layer F.Cu) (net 11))
 (segment (start 89.779 99.46) (end 92.7635 99.46) (width 0.2) (layer F.Cu) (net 11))
 (segment (start 88.509 98.19) (end 88.5725 98.19) (width 0.2) (layer F.Cu) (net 11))
 (segment (start 91.049 98.19) (end 89.779 96.92) (width 0.2) (layer F.Cu) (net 12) (status 400000))
 (segment (start 85.207 99.417) (end 83.64 100.984) (width 0.2) (layer F.Cu) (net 12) (status 800000))
 (segment (start 85.207 98.5075) (end 85.207 99.417) (width 0.2) (layer F.Cu) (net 12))
 (segment (start 86.7945 96.92) (end 85.207 98.5075) (width 0.2) (layer F.Cu) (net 12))
 (segment (start 89.779 96.92) (end 86.7945 96.92) (width 0.2) (layer F.Cu) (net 12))
 (segment (start 91.049 98.19) (end 93.97 98.19) (width 0.2) (layer F.Cu) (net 12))
 (segment (start 94.6076 98.8276) (end 97.2102 98.8276) (width 0.2) (layer F.Cu) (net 12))
 (segment (start 93.97 98.19) (end 94.6076 98.8276) (width 0.2) (layer F.Cu) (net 12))
 (segment (start 83.64 98.444) (end 83.8735 98.444) (width 0.2) (layer F.Cu) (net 15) (status C00000))
 (segment (start 83.8735 98.444) (end 86.477 95.8405) (width 0.2) (layer F.Cu) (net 15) (status 400000))
 (segment (start 86.477 95.8405) (end 86.477 93.8085) (width 0.2) (layer F.Cu) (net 15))
 (segment (start 86.477 93.8085) (end 87.1755 93.11) (width 0.2) (layer F.Cu) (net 15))
 (segment (start 87.1755 93.11) (end 88.509 93.11) (width 0.2) (layer F.Cu) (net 15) (status 800000))
 (segment (start 88.509 93.11) (end 88.509 93.1735) (width 0.2) (layer F.Cu) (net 15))
 (segment (start 88.509 93.1735) (end 89.7155 94.38) (width 0.2) (layer F.Cu) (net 15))
 (segment (start 89.7155 94.38) (end 92.7 94.38) (width 0.2) (layer F.Cu) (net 15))
 (segment (start 92.7 94.38) (end 93.589 95.269) (width 0.2) (layer F.Cu) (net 15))
 (segment (start 93.589 95.269) (end 93.589 96.6025) (width 0.2) (layer F.Cu) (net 15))
 (segment (start 93.589 96.6025) (end 95.3141 98.3276) (width 0.2) (layer F.Cu) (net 15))
 (segment (start 95.3141 98.3276) (end 97.2102 98.3276) (width 0.2) (layer F.Cu) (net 15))
 (segment (start 91.049 93.11) (end 90.287 93.11) (width 0.2) (layer F.Cu) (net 16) (status C00000))
 (segment (start 90.287 93.11) (end 89.779 92.602) (width 0.2) (layer F.Cu) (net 16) (status 400000))
 (segment (start 85.588 93.956) (end 83.64 95.904) (width 0.2) (layer F.Cu) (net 16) (status 800000))
 (segment (start 85.588 93.0465) (end 85.588 93.956) (width 0.2) (layer F.Cu) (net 16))
 (segment (start 86.7945 91.84) (end 85.588 93.0465) (width 0.2) (layer F.Cu) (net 16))
 (segment (start 89.398 91.84) (end 86.7945 91.84) (width 0.2) (layer F.Cu) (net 16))
 (segment (start 89.779 92.221) (end 89.398 91.84) (width 0.2) (layer F.Cu) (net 16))
 (segment (start 89.779 92.602) (end 89.779 92.221) (width 0.2) (layer F.Cu) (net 16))
 (segment (start 91.049 93.11) (end 90.8585 93.11) (width 0.2) (layer F.Cu) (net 16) (status C00000))
 (segment (start 97.2102 97.3276) (end 95.5206 97.3276) (width 0.2) (layer F.Cu) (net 16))
 (segment (start 92.5095 93.11) (end 91.049 93.11) (width 0.2) (layer F.Cu) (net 16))
 (segment (start 94.351 94.9515) (end 92.5095 93.11) (width 0.2) (layer F.Cu) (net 16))
 (segment (start 94.351 96.158) (end 94.351 94.9515) (width 0.2) (layer F.Cu) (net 16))
 (segment (start 95.5206 97.3276) (end 94.351 96.158) (width 0.2) (layer F.Cu) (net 16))
 (segment (start 83.64 93.364) (end 84.2545 93.364) (width 0.2) (layer F.Cu) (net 17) (status 400000))
 (segment (start 87.0485 90.57) (end 88.509 90.57) (width 0.2) (layer F.Cu) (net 17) (status 800000))
 (segment (start 84.2545 93.364) (end 87.0485 90.57) (width 0.2) (layer F.Cu) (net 17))
 (segment (start 89.017 90.57) (end 90.287 91.84) (width 0.2) (layer F.Cu) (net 17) (status 400000))
 (segment (start 96.1636 96.8276) (end 97.2102 96.8276) (width 0.2) (layer F.Cu) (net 17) (status 800000))
 (segment (start 95.0495 95.7135) (end 96.1636 96.8276) (width 0.2) (layer F.Cu) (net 17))
 (segment (start 95.0495 94.1895) (end 95.0495 95.7135) (width 0.2) (layer F.Cu) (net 17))
 (segment (start 92.7 91.84) (end 95.0495 94.1895) (width 0.2) (layer F.Cu) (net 17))
 (segment (start 90.287 91.84) (end 92.7 91.84) (width 0.2) (layer F.Cu) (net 17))
 (segment (start 84.1275 93.364) (end 83.64 93.364) (width 0.2) (layer F.Cu) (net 17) (status C00000))
 (segment (start 86.5405 89.3) (end 85.9055 89.3) (width 0.2) (layer F.Cu) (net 18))
 (segment (start 89.9695 89.3) (end 86.5405 89.3) (width 0.2) (layer F.Cu) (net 18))
 (segment (start 91.049 90.3795) (end 89.9695 89.3) (width 0.2) (layer F.Cu) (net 18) (status 400000))
 (segment (start 84.3815 90.824) (end 83.64 90.824) (width 0.2) (layer F.Cu) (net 18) (status 800000))
 (segment (start 85.9055 89.3) (end 84.3815 90.824) (width 0.2) (layer F.Cu) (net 18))
 (segment (start 91.049 90.57) (end 91.049 90.3795) (width 0.2) (layer F.Cu) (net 18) (status C00000))
 (segment (start 97.2102 95.8276) (end 97.2102 94.8262) (width 0.2) (layer F.Cu) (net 18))
 (segment (start 92.954 90.57) (end 91.049 90.57) (width 0.2) (layer F.Cu) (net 18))
 (segment (start 97.2102 94.8262) (end 92.954 90.57) (width 0.2) (layer F.Cu) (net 18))
 (segment (start 97.2102 95.8276) (end 96.3066 95.8276) (width 0.2) (layer F.Cu) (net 18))
 (segment (start 97.1448 95.8276) (end 97.2102 95.8276) (width 0.3) (layer F.Cu) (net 18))
 (segment (start 63.1344 90.9048) (end 63.1344 90.8621) (width 0.2) (layer F.Cu) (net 25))
 (segment (start 63.1344 90.8621) (end 64.125 89.8715) (width 0.2) (layer F.Cu) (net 25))
 (segment (start 64.125 89.8715) (end 75.2375 89.8715) (width 0.2) (layer F.Cu) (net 25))
 (segment (start 75.2375 89.8715) (end 84.699 80.41) (width 0.2) (layer F.Cu) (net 25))
 (segment (start 84.699 80.41) (end 88.509 80.41) (width 0.2) (layer F.Cu) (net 25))
 (segment (start 91.049 80.41) (end 89.779 81.68) (width 0.2) (layer F.Cu) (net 26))
 (segment (start 75.9822 90.9048) (end 65.1344 90.9048) (width 0.2) (layer F.Cu) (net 26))
 (segment (start 85.207 81.68) (end 75.9822 90.9048) (width 0.2) (layer F.Cu) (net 26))
 (segment (start 89.779 81.68) (end 85.207 81.68) (width 0.2) (layer F.Cu) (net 26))
 (segment (start 65.1344 90.9048) (end 64.5776 90.9048) (width 0.3) (layer F.Cu) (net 26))
 (segment (start 63.1344 86.9048) (end 63.1344 86.9124) (width 0.2) (layer F.Cu) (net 28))
 (segment (start 63.1344 86.9124) (end 64.125 87.903) (width 0.2) (layer F.Cu) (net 28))
 (segment (start 64.125 87.903) (end 74.2215 87.903) (width 0.2) (layer F.Cu) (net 28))
 (segment (start 74.2215 87.903) (end 85.5245 76.6) (width 0.2) (layer F.Cu) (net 28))
 (segment (start 85.5245 76.6) (end 89.779 76.6) (width 0.2) (layer F.Cu) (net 28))
 (segment (start 89.779 76.6) (end 91.049 77.87) (width 0.2) (layer F.Cu) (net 28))
 (segment (start 65.1344 86.9048) (end 71.6637 86.9048) (width 0.2) (layer F.Cu) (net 29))
 (segment (start 83.2385 75.33) (end 88.509 75.33) (width 0.2) (layer F.Cu) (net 29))
 (segment (start 71.6637 86.9048) (end 83.2385 75.33) (width 0.2) (layer F.Cu) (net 29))
 (segment (start 63.1344 84.9048) (end 63.1344 84.8931) (width 0.2) (layer F.Cu) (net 30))
 (segment (start 63.1344 84.8931) (end 64.125 83.9025) (width 0.2) (layer F.Cu) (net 30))
 (segment (start 89.779 74.06) (end 91.049 75.33) (width 0.2) (layer F.Cu) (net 30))
 (segment (start 89.779 72.028) (end 89.779 74.06) (width 0.2) (layer F.Cu) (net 30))
 (segment (start 89.271 71.52) (end 89.779 72.028) (width 0.2) (layer F.Cu) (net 30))
 (segment (start 82.794 71.52) (end 89.271 71.52) (width 0.2) (layer F.Cu) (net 30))
 (segment (start 70.4115 83.9025) (end 82.794 71.52) (width 0.2) (layer F.Cu) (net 30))
 (segment (start 64.125 83.9025) (end 70.4115 83.9025) (width 0.2) (layer F.Cu) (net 30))
 (segment (start 65.1344 84.9048) (end 71.0602 84.9048) (width 0.2) (layer F.Cu) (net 31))
 (segment (start 83.175 72.79) (end 88.509 72.79) (width 0.2) (layer F.Cu) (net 31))
 (segment (start 71.0602 84.9048) (end 83.175 72.79) (width 0.2) (layer F.Cu) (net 31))
 (segment (start 65.1344 84.9048) (end 64.7356 84.9048) (width 0.3) (layer F.Cu) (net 31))
 (segment (start 63.1344 82.9048) (end 63.1542 82.9048) (width 0.2) (layer F.Cu) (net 32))
 (segment (start 63.1542 82.9048) (end 64.1885 81.8705) (width 0.2) (layer F.Cu) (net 32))
 (segment (start 64.1885 81.8705) (end 68.189 81.8705) (width 0.2) (layer F.Cu) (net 32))
 (segment (start 68.189 81.8705) (end 81.0795 68.98) (width 0.2) (layer F.Cu) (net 32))
 (segment (start 81.0795 68.98) (end 91.811 68.98) (width 0.2) (layer F.Cu) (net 32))
 (segment (start 91.811 68.98) (end 92.7 69.869) (width 0.2) (layer F.Cu) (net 32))
 (segment (start 92.7 69.869) (end 92.7 71.139) (width 0.2) (layer F.Cu) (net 32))
 (segment (start 92.7 71.139) (end 91.049 72.79) (width 0.2) (layer F.Cu) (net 32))
 (segment (start 65.1344 82.9048) (end 69.1232 82.9048) (width 0.2) (layer F.Cu) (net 33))
 (segment (start 81.778 70.25) (end 88.509 70.25) (width 0.2) (layer F.Cu) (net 33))
 (segment (start 69.1232 82.9048) (end 81.778 70.25) (width 0.2) (layer F.Cu) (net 33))
 (segment (start 63.1344 92.9048) (end 63.1344 92.8941) (width 0.2) (layer F.Cu) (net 23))
 (segment (start 63.1344 92.8941) (end 64.125 91.9035) (width 0.2) (layer F.Cu) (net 23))
 (segment (start 64.125 91.9035) (end 76.952 91.9035) (width 0.2) (layer F.Cu) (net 23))
 (segment (start 76.952 91.9035) (end 85.9055 82.95) (width 0.2) (layer F.Cu) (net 23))
 (segment (start 85.9055 82.95) (end 88.509 82.95) (width 0.2) (layer F.Cu) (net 23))
 (segment (start 91.049 82.95) (end 90.9855 82.95) (width 0.2) (layer F.Cu) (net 24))
 (segment (start 90.9855 82.95) (end 89.7155 84.22) (width 0.2) (layer F.Cu) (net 24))
 (segment (start 89.7155 84.22) (end 86.0325 84.22) (width 0.2) (layer F.Cu) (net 24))
 (segment (start 86.0325 84.22) (end 77.3477 92.9048) (width 0.2) (layer F.Cu) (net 24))
 (segment (start 77.3477 92.9048) (end 65.1344 92.9048) (width 0.2) (layer F.Cu) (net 24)))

